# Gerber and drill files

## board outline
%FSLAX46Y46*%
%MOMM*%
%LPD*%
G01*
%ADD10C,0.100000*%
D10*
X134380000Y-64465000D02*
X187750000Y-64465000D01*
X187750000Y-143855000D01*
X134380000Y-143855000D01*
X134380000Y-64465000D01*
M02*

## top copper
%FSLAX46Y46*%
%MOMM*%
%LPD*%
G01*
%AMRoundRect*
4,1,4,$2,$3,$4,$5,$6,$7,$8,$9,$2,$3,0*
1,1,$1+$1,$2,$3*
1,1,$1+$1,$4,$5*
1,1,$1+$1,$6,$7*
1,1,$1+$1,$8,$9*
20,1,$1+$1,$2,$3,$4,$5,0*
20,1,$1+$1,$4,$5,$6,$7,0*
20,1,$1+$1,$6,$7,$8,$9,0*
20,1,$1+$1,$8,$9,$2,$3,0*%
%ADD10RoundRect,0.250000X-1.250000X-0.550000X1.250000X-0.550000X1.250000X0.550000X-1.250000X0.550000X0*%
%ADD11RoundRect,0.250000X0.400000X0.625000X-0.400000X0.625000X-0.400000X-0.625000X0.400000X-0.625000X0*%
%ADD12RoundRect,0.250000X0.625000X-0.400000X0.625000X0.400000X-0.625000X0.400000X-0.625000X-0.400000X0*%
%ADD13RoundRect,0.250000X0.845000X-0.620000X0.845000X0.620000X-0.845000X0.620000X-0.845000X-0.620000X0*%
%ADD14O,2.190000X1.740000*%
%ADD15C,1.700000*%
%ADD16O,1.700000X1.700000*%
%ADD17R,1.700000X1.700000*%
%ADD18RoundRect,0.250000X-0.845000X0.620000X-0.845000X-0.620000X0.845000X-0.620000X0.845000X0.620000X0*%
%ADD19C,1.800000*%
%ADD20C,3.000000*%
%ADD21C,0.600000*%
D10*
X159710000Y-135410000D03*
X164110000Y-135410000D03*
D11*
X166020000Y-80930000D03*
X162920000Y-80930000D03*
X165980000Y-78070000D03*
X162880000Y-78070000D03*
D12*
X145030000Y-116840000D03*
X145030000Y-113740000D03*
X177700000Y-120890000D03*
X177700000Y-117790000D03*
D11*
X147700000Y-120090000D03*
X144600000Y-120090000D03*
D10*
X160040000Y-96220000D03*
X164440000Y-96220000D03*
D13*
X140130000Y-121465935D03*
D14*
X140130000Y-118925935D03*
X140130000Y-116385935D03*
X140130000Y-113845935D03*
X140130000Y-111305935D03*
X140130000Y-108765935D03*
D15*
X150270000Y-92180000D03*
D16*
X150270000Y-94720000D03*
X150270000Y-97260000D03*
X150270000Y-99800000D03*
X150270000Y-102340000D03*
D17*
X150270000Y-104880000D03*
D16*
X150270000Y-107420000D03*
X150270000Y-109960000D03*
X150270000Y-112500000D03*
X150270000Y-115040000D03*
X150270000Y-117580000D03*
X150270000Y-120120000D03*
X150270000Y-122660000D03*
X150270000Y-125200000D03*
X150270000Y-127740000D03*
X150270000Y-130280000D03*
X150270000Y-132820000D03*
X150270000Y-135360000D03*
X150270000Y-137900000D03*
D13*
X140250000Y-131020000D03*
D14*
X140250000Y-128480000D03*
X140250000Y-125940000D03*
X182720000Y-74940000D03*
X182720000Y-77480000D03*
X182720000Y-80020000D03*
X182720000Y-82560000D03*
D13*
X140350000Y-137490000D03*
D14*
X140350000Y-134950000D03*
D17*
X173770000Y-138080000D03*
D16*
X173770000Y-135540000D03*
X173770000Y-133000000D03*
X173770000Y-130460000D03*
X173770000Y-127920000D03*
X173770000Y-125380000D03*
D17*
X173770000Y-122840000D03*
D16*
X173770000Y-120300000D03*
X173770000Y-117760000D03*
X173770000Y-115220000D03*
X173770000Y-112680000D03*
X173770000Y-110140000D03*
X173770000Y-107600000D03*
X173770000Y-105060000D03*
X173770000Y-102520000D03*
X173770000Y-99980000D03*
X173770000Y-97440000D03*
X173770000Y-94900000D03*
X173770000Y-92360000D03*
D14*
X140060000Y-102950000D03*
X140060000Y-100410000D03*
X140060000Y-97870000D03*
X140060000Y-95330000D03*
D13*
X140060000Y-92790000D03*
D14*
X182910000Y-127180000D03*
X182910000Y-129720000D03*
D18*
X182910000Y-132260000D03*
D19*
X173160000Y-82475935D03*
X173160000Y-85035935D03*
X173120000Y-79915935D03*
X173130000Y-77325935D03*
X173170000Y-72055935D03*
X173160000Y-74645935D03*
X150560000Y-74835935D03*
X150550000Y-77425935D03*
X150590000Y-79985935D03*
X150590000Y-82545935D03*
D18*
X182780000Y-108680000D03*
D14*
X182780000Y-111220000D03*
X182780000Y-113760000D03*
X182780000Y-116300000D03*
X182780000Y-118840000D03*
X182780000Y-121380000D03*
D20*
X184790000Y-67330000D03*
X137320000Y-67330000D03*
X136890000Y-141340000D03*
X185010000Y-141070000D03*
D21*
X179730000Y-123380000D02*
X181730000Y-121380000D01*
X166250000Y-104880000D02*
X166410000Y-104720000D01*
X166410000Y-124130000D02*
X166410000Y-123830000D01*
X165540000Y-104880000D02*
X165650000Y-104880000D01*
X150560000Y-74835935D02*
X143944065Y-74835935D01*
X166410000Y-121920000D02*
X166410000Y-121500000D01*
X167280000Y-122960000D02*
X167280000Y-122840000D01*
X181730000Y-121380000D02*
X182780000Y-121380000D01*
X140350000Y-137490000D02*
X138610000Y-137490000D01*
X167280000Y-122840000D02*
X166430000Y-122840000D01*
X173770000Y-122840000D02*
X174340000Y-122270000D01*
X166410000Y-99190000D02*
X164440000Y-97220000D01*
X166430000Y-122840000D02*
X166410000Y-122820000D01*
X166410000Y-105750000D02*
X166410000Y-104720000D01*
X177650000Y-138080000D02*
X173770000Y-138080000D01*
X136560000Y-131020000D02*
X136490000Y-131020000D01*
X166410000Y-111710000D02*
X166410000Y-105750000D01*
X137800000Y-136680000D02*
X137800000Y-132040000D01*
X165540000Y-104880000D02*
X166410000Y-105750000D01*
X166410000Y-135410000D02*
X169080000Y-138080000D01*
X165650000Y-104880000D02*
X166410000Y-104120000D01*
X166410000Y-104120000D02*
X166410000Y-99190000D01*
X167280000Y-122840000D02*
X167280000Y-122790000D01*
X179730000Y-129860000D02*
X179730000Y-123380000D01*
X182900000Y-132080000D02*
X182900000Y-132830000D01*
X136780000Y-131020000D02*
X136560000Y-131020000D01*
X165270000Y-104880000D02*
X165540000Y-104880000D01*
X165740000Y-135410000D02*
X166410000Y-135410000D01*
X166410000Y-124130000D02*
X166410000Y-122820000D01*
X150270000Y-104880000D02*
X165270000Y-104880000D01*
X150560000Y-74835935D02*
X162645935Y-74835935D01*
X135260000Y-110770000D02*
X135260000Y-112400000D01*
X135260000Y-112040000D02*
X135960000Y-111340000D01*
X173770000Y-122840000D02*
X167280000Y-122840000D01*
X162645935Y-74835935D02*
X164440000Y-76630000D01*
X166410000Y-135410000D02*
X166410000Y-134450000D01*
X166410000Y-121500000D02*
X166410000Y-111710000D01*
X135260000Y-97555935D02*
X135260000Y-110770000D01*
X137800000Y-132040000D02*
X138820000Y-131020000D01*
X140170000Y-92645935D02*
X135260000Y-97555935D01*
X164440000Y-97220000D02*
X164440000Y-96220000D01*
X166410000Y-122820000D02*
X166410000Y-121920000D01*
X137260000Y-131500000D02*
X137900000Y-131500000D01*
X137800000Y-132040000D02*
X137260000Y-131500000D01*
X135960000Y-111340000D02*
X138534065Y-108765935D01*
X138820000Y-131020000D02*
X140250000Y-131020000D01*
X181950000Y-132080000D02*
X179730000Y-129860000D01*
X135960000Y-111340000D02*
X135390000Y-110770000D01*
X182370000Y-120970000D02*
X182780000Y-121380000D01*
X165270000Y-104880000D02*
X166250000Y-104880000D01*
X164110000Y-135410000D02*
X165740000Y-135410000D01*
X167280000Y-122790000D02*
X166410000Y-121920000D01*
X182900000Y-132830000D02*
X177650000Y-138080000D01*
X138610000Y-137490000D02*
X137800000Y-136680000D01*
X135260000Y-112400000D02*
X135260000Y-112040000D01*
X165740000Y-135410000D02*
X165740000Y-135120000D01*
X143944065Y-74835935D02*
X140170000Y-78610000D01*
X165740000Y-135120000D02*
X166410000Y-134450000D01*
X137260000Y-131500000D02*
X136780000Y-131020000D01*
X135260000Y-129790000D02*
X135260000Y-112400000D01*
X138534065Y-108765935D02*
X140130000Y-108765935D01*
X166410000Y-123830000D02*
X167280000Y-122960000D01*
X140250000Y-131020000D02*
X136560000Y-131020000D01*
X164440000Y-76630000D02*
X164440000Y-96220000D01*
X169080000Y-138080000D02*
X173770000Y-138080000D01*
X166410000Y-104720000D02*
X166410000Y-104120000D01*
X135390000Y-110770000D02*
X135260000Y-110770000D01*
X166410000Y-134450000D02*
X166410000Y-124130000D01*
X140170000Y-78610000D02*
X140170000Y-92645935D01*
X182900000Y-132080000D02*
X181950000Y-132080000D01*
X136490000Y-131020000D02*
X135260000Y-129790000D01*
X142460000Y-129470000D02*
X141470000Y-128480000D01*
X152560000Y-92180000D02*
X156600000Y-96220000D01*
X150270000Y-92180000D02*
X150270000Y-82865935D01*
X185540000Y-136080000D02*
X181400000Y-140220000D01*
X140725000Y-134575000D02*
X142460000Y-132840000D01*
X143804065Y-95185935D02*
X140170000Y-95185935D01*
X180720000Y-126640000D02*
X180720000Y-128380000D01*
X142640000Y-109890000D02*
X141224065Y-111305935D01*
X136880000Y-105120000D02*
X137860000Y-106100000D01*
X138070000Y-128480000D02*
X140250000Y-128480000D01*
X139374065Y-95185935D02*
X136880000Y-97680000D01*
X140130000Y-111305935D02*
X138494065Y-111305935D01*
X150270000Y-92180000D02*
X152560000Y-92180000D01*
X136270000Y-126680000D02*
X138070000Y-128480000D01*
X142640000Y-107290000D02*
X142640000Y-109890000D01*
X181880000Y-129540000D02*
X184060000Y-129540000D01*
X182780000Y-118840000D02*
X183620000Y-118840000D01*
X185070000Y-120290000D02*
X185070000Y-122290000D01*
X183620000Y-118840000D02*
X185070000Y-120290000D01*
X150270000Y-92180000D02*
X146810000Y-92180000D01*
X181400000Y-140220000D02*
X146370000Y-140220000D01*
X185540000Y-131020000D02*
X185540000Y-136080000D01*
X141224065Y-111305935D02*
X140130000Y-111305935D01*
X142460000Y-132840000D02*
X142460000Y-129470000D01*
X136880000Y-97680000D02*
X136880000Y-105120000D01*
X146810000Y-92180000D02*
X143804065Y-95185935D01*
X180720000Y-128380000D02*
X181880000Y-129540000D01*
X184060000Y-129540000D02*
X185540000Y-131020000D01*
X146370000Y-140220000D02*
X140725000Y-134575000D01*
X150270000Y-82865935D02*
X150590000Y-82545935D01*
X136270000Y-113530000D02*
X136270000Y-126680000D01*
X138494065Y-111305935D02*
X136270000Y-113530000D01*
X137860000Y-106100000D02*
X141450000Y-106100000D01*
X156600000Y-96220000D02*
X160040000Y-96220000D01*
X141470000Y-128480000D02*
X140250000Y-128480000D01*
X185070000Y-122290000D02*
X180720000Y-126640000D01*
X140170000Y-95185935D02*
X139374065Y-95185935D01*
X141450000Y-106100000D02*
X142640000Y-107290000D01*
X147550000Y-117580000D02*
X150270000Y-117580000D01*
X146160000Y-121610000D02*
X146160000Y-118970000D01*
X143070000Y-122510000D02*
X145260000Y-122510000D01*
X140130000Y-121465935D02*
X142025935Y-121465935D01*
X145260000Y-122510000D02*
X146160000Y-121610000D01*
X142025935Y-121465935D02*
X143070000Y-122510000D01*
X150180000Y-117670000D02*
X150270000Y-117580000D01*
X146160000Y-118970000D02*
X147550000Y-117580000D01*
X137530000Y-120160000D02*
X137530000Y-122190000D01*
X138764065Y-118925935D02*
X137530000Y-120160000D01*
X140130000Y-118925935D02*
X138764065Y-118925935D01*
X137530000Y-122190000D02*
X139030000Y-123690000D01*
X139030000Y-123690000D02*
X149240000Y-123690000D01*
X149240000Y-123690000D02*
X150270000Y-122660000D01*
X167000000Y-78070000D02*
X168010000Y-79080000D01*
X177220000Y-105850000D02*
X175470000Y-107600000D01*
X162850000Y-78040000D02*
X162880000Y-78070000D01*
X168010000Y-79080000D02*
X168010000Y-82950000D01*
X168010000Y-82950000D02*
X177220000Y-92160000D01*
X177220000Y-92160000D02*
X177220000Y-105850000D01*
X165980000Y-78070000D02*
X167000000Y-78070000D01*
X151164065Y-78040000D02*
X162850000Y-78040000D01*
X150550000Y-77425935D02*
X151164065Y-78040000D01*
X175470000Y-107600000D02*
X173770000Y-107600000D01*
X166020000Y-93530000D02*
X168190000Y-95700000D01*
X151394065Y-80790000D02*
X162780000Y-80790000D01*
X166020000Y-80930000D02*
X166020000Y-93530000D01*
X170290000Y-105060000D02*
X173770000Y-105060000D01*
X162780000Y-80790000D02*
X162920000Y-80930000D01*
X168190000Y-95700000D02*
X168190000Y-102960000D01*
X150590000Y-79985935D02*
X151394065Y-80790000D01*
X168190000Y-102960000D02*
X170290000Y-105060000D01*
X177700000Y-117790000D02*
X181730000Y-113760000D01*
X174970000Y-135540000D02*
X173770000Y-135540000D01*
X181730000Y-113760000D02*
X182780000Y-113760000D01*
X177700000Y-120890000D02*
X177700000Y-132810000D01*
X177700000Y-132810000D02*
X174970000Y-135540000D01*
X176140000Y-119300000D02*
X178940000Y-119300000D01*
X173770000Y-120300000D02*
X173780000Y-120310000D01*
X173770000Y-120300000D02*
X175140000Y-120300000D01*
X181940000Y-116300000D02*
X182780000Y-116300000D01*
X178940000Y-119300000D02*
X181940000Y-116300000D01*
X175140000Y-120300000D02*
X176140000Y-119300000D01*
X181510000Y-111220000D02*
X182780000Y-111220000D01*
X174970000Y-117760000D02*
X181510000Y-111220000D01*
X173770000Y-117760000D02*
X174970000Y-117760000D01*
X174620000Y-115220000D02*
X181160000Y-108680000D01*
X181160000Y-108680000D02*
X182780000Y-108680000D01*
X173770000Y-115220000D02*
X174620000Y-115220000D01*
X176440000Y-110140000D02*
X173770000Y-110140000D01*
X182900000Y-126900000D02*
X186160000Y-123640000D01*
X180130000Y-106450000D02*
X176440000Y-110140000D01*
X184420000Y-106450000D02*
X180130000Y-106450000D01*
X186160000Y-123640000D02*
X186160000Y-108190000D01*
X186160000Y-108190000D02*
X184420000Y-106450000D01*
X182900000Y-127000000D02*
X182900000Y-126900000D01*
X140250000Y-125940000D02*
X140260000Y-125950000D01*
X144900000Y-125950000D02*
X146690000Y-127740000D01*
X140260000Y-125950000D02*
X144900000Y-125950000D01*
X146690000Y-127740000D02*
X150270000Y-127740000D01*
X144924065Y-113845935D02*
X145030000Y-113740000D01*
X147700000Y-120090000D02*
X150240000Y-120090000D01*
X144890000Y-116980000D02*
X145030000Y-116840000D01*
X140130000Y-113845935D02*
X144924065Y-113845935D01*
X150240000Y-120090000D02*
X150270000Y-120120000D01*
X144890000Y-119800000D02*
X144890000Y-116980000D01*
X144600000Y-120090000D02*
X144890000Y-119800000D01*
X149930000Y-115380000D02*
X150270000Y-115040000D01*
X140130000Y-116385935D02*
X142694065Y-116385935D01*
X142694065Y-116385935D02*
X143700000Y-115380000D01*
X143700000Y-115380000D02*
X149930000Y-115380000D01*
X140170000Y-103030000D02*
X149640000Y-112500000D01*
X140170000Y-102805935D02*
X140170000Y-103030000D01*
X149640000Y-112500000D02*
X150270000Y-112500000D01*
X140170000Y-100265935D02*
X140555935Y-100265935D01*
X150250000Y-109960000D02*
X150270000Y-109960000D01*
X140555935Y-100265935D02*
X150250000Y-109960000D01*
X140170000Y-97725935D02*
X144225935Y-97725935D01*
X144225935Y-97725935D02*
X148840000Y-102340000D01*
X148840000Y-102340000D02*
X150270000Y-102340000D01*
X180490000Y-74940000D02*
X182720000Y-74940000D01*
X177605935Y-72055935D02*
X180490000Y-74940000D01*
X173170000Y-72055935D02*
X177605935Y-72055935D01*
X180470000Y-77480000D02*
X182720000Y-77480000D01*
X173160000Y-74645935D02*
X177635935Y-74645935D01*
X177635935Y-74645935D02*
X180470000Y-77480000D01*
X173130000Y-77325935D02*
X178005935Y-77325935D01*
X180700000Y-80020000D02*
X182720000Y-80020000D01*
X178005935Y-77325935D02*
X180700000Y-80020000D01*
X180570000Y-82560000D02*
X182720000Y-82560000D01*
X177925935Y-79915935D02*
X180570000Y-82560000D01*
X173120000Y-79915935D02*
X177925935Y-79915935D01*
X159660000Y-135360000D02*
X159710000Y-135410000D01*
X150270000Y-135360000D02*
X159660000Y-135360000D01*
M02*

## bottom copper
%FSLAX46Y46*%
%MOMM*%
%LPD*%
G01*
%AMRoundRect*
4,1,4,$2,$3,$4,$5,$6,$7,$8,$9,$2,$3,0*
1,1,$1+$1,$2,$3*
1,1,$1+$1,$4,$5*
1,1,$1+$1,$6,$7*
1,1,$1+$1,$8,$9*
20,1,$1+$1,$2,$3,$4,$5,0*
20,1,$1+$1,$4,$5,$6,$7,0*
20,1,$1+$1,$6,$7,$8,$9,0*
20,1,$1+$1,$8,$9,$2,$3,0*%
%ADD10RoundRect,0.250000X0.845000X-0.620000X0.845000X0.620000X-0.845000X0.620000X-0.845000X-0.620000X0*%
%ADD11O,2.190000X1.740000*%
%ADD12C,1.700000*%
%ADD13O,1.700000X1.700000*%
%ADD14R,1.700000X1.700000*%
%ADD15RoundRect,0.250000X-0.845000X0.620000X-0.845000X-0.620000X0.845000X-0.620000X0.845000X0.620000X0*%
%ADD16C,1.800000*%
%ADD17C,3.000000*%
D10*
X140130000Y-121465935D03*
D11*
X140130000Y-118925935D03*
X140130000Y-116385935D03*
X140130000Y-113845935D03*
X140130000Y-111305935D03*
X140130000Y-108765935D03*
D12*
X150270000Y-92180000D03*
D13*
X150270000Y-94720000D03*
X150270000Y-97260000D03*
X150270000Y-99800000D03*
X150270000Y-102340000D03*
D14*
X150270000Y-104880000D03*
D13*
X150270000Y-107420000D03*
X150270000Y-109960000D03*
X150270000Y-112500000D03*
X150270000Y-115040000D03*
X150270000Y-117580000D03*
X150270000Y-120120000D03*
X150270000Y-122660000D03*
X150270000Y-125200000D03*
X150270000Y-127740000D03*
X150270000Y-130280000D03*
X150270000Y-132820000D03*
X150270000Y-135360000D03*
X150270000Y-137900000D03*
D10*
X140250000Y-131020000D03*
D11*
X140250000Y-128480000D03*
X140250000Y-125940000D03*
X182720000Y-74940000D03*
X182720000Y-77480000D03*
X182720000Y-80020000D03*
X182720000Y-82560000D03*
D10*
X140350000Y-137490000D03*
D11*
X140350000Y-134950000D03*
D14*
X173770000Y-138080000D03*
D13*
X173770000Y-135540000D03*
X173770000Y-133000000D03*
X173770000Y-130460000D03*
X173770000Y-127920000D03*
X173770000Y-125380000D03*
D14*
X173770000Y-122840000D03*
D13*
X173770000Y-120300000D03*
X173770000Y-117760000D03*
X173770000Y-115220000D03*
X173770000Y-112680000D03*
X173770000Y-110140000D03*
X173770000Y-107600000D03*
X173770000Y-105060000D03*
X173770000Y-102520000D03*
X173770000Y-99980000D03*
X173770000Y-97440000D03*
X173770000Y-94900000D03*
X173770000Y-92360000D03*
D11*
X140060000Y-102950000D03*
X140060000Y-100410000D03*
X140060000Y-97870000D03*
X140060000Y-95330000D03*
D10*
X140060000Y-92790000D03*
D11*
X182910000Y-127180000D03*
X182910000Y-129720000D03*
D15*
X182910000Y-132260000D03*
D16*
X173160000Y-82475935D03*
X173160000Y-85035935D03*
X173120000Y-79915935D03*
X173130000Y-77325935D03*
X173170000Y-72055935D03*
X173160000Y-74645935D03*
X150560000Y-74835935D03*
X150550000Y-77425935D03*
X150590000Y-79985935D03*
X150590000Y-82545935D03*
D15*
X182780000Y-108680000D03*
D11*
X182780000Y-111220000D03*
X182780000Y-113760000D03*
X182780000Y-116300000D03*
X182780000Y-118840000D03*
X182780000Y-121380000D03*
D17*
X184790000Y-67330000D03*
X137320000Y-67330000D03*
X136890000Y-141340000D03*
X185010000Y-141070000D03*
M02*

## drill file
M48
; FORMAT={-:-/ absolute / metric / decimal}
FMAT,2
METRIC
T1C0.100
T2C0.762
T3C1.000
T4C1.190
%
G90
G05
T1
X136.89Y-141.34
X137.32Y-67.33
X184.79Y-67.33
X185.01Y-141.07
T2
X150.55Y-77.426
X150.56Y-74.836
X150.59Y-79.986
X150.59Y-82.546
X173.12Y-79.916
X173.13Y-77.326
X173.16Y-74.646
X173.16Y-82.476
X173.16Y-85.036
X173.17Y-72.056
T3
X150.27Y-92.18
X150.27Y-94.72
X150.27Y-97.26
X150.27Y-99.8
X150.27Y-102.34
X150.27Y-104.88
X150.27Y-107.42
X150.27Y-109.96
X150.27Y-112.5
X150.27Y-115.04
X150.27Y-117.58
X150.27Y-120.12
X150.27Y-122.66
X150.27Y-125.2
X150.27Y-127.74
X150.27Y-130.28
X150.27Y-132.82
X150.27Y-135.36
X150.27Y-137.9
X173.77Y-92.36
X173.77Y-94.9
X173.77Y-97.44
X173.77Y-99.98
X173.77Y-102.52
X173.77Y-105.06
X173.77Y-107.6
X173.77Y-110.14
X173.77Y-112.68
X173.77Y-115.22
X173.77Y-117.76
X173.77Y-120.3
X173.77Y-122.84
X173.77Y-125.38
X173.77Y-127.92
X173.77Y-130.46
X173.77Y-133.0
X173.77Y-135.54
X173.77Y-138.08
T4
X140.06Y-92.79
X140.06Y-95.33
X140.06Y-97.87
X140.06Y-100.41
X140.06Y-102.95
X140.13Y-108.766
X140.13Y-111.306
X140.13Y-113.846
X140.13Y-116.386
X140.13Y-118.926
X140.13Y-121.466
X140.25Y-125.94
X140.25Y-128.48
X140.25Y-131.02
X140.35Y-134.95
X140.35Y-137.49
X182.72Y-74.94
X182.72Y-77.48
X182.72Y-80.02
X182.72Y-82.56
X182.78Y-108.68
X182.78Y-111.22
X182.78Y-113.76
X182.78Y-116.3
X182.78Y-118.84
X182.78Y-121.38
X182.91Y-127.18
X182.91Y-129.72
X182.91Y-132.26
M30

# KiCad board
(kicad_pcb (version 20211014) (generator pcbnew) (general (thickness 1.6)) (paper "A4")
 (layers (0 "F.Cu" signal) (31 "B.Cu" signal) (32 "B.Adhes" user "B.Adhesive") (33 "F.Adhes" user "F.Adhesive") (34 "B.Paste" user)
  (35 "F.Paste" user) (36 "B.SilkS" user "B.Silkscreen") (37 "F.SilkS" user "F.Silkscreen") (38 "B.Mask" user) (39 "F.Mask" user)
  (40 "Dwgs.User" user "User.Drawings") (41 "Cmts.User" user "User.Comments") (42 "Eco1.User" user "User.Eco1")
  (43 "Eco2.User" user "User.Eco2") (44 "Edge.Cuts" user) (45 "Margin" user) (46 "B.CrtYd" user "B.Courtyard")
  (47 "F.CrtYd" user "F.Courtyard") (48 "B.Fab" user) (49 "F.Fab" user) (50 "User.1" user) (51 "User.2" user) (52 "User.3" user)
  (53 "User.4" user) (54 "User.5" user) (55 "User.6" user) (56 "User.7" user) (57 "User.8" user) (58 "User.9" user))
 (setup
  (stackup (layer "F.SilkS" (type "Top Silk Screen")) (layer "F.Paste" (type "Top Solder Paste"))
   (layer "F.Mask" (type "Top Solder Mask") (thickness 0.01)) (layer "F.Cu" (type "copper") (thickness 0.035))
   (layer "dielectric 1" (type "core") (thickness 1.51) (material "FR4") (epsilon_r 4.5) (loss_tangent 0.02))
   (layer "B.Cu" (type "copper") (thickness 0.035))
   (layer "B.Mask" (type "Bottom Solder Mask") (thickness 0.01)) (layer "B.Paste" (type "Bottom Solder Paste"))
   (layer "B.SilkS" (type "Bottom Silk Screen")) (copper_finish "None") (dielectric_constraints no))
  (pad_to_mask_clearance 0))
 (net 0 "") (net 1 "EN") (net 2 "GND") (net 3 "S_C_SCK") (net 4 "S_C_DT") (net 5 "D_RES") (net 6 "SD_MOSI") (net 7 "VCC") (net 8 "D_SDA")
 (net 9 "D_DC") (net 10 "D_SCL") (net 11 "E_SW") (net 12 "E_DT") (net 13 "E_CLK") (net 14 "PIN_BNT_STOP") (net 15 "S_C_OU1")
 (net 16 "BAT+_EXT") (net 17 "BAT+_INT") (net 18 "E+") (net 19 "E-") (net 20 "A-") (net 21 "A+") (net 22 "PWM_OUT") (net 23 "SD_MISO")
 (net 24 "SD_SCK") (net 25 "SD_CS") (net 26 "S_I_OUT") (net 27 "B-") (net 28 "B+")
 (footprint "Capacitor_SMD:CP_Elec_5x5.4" (layer "F.Cu") (at 161.91 135.41)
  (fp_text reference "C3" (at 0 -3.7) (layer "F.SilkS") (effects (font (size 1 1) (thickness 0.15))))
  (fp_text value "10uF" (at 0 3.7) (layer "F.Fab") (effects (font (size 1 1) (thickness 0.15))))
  (pad "1" smd roundrect (at -2.2 0) (size 3 1.6) (layers "F.Cu" "F.Paste" "F.Mask") (roundrect_rratio 0.15625) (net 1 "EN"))
  (pad "2" smd roundrect (at 2.2 0) (size 3 1.6) (layers "F.Cu" "F.Paste" "F.Mask") (roundrect_rratio 0.15625) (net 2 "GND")))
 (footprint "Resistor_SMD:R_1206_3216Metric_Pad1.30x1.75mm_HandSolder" (layer "F.Cu") (at 164.47 80.93 180)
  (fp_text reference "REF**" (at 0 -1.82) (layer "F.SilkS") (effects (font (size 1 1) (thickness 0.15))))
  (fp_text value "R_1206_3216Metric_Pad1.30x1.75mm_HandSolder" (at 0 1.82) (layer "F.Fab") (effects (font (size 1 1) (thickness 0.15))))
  (pad "1" smd roundrect (at -1.55 0 180) (size 1.3 1.75) (layers "F.Cu" "F.Paste" "F.Mask") (roundrect_rratio 0.192308) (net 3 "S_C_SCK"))
  (pad "2" smd roundrect (at 1.55 0 180) (size 1.3 1.75) (layers "F.Cu" "F.Paste" "F.Mask") (roundrect_rratio 0.192308) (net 3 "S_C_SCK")))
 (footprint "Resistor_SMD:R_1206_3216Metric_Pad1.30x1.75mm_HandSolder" (layer "F.Cu") (at 164.43 78.07 180)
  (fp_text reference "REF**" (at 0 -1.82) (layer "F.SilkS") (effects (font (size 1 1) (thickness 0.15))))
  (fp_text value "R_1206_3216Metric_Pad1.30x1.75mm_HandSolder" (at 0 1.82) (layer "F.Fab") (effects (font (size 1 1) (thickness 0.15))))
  (pad "1" smd roundrect (at -1.55 0 180) (size 1.3 1.75) (layers "F.Cu" "F.Paste" "F.Mask") (roundrect_rratio 0.192308) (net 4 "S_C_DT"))
  (pad "2" smd roundrect (at 1.55 0 180) (size 1.3 1.75) (layers "F.Cu" "F.Paste" "F.Mask") (roundrect_rratio 0.192308) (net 4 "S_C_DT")))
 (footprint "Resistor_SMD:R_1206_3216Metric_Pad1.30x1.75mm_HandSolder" (layer "F.Cu") (at 145.03 115.29 90)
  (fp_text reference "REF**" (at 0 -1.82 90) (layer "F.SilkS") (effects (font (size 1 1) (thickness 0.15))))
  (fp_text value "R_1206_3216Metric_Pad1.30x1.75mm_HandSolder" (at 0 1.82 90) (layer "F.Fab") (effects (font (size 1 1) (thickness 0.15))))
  (pad "1" smd roundrect (at -1.55 0 90) (size 1.3 1.75) (layers "F.Cu" "F.Paste" "F.Mask") (roundrect_rratio 0.192308) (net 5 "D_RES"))
  (pad "2" smd roundrect (at 1.55 0 90) (size 1.3 1.75) (layers "F.Cu" "F.Paste" "F.Mask") (roundrect_rratio 0.192308) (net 5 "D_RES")))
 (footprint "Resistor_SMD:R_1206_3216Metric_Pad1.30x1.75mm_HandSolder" (layer "F.Cu") (at 177.7 119.34 90)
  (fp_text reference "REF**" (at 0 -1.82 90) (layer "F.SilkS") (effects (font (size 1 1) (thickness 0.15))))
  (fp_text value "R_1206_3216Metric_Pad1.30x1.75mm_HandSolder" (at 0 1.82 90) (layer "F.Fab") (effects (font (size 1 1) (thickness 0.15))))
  (pad "1" smd roundrect (at -1.55 0 90) (size 1.3 1.75) (layers "F.Cu" "F.Paste" "F.Mask") (roundrect_rratio 0.192308) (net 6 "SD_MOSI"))
  (pad "2" smd roundrect (at 1.55 0 90) (size 1.3 1.75) (layers "F.Cu" "F.Paste" "F.Mask") (roundrect_rratio 0.192308) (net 6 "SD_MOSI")))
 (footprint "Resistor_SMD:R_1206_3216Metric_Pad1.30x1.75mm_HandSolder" (layer "F.Cu") (at 146.15 120.09 180)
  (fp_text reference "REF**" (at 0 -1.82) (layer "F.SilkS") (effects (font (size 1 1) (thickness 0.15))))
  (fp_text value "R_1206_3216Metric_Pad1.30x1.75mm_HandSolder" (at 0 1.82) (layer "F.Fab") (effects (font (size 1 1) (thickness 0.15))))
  (pad "1" smd roundrect (at -1.55 0 180) (size 1.3 1.75) (layers "F.Cu" "F.Paste" "F.Mask") (roundrect_rratio 0.192308) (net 5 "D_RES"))
  (pad "2" smd roundrect (at 1.55 0 180) (size 1.3 1.75) (layers "F.Cu" "F.Paste" "F.Mask") (roundrect_rratio 0.192308) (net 5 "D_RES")))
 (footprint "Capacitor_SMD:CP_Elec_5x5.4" (layer "F.Cu") (at 162.24 96.22)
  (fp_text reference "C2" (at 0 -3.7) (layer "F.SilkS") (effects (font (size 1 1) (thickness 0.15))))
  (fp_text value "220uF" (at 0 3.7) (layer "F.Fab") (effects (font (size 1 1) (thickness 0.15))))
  (pad "1" smd roundrect (at -2.2 0) (size 3 1.6) (layers "F.Cu" "F.Paste" "F.Mask") (roundrect_rratio 0.15625) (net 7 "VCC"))
  (pad "2" smd roundrect (at 2.2 0) (size 3 1.6) (layers "F.Cu" "F.Paste" "F.Mask") (roundrect_rratio 0.15625) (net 2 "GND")))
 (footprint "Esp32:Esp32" (layer "F.Cu") (at 162.18 114.97)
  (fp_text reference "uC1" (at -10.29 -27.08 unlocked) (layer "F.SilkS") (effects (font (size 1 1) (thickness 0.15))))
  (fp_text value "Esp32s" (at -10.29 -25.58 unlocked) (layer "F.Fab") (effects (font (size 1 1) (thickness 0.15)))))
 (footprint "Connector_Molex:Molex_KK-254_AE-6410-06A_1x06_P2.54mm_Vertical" (layer "B.Cu") (at 140.13 121.465935 90)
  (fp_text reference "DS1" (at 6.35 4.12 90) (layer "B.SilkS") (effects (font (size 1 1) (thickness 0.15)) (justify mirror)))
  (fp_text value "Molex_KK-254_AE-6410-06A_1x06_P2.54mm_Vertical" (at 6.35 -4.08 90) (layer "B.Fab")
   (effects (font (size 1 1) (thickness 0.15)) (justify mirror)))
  (pad "1" thru_hole roundrect (at 0 0 90) (size 1.74 2.19) (drill 1.19) (layers *.Cu *.Mask) (roundrect_rratio 0.143678) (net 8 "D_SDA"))
  (pad "2" thru_hole oval (at 2.54 0 90) (size 1.74 2.19) (drill 1.19) (layers *.Cu *.Mask) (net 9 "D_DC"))
  (pad "3" thru_hole oval (at 5.08 0 90) (size 1.74 2.19) (drill 1.19) (layers *.Cu *.Mask) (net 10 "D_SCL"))
  (pad "4" thru_hole oval (at 7.62 0 90) (size 1.74 2.19) (drill 1.19) (layers *.Cu *.Mask) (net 5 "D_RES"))
  (pad "5" thru_hole oval (at 10.16 0 90) (size 1.74 2.19) (drill 1.19) (layers *.Cu *.Mask) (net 7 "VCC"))
  (pad "6" thru_hole oval (at 12.7 0 90) (size 1.74 2.19) (drill 1.19) (layers *.Cu *.Mask) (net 2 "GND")))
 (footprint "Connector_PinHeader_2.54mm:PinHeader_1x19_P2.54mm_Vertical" (layer "B.Cu") (at 150.27 92.18 180)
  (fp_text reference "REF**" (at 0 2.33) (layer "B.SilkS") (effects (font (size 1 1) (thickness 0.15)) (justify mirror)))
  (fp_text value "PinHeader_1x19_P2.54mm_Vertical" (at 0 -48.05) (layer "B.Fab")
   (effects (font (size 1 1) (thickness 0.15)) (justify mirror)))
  (pad "1" thru_hole circle (at 0 0 180) (size 1.7 1.7) (drill 1) (layers *.Cu *.Mask) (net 7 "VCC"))
  (pad "2" thru_hole oval (at 0 -2.54 180) (size 1.7 1.7) (drill 1) (layers *.Cu *.Mask))
  (pad "3" thru_hole oval (at 0 -5.08 180) (size 1.7 1.7) (drill 1) (layers *.Cu *.Mask))
  (pad "4" thru_hole oval (at 0 -7.62 180) (size 1.7 1.7) (drill 1) (layers *.Cu *.Mask))
  (pad "5" thru_hole oval (at 0 -10.16 180) (size 1.7 1.7) (drill 1) (layers *.Cu *.Mask) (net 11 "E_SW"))
  (pad "6" thru_hole rect (at 0 -12.7 180) (size 1.7 1.7) (drill 1) (layers *.Cu *.Mask) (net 2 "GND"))
  (pad "7" thru_hole oval (at 0 -15.24 180) (size 1.7 1.7) (drill 1) (layers *.Cu *.Mask))
  (pad "8" thru_hole oval (at 0 -17.78 180) (size 1.7 1.7) (drill 1) (layers *.Cu *.Mask) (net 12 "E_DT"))
  (pad "9" thru_hole oval (at 0 -20.32 180) (size 1.7 1.7) (drill 1) (layers *.Cu *.Mask) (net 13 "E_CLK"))
  (pad "10" thru_hole oval (at 0 -22.86 180) (size 1.7 1.7) (drill 1) (layers *.Cu *.Mask) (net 10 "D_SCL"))
  (pad "11" thru_hole oval (at 0 -25.4 180) (size 1.7 1.7) (drill 1) (layers *.Cu *.Mask) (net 8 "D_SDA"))
  (pad "12" thru_hole oval (at 0 -27.94 180) (size 1.7 1.7) (drill 1) (layers *.Cu *.Mask) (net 5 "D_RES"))
  (pad "13" thru_hole oval (at 0 -30.48 180) (size 1.7 1.7) (drill 1) (layers *.Cu *.Mask) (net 9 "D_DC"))
  (pad "14" thru_hole oval (at 0 -33.02 180) (size 1.7 1.7) (drill 1) (layers *.Cu *.Mask) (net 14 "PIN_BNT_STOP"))
  (pad "15" thru_hole oval (at 0 -35.56 180) (size 1.7 1.7) (drill 1) (layers *.Cu *.Mask) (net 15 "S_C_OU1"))
  (pad "16" thru_hole oval (at 0 -38.1 180) (size 1.7 1.7) (drill 1) (layers *.Cu *.Mask) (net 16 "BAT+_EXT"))
  (pad "17" thru_hole oval (at 0 -40.64 180) (size 1.7 1.7) (drill 1) (layers *.Cu *.Mask) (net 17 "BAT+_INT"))
  (pad "18" thru_hole oval (at 0 -43.18 180) (size 1.7 1.7) (drill 1) (layers *.Cu *.Mask) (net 1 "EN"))
  (pad "19" thru_hole oval (at 0 -45.72 180) (size 1.7 1.7) (drill 1) (layers *.Cu *.Mask)))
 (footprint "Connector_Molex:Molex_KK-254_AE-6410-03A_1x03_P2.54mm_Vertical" (layer "B.Cu") (at 140.25 131.02 90)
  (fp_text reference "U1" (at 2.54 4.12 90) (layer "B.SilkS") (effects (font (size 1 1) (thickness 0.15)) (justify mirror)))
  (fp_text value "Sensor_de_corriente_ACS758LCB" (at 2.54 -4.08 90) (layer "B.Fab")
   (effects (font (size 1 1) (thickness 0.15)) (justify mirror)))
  (pad "1" thru_hole roundrect (at 0 0 90) (size 1.74 2.19) (drill 1.19) (layers *.Cu *.Mask) (roundrect_rratio 0.143678) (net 2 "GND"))
  (pad "2" thru_hole oval (at 2.54 0 90) (size 1.74 2.19) (drill 1.19) (layers *.Cu *.Mask) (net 7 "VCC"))
  (pad "3" thru_hole oval (at 5.08 0 90) (size 1.74 2.19) (drill 1.19) (layers *.Cu *.Mask) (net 15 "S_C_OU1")))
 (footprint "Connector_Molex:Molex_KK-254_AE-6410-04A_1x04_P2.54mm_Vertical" (layer "B.Cu") (at 182.72 74.94 -90)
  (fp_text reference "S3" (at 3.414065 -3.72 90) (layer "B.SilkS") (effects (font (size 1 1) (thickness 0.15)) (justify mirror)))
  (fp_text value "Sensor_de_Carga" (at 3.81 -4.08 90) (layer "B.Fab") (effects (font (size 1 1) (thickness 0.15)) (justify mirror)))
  (pad "1" thru_hole oval (at 0 0 270) (size 1.74 2.19) (drill 1.19) (layers *.Cu *.Mask) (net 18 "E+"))
  (pad "2" thru_hole oval (at 2.54 0 270) (size 1.74 2.19) (drill 1.19) (layers *.Cu *.Mask) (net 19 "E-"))
  (pad "3" thru_hole oval (at 5.08 0 270) (size 1.74 2.19) (drill 1.19) (layers *.Cu *.Mask) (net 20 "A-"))
  (pad "4" thru_hole oval (at 7.62 0 270) (size 1.74 2.19) (drill 1.19) (layers *.Cu *.Mask) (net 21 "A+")))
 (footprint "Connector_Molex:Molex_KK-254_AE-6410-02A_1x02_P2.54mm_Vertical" (layer "B.Cu") (at 140.35 137.49 90)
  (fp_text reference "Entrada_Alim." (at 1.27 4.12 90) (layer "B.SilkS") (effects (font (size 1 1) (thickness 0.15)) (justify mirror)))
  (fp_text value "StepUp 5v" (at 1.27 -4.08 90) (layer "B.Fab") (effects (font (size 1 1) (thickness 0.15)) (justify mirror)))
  (pad "1" thru_hole roundrect (at 0 0 90) (size 1.74 2.19) (drill 1.19) (layers *.Cu *.Mask) (roundrect_rratio 0.143678) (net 2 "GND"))
  (pad "2" thru_hole oval (at 2.54 0 90) (size 1.74 2.19) (drill 1.19) (layers *.Cu *.Mask) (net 7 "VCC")))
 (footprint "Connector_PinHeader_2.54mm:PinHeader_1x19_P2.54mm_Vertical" (layer "B.Cu") (at 173.77 138.08)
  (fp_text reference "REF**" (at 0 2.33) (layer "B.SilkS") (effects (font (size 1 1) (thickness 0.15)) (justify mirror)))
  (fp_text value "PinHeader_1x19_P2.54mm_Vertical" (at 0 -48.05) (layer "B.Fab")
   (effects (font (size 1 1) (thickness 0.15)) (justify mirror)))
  (pad "1" thru_hole rect (at 0 0) (size 1.7 1.7) (drill 1) (layers *.Cu *.Mask) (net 2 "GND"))
  (pad "2" thru_hole oval (at 0 -2.54) (size 1.7 1.7) (drill 1) (layers *.Cu *.Mask) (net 6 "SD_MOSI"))
  (pad "3" thru_hole oval (at 0 -5.08) (size 1.7 1.7) (drill 1) (layers *.Cu *.Mask) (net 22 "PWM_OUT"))
  (pad "4" thru_hole oval (at 0 -7.62) (size 1.7 1.7) (drill 1) (layers *.Cu *.Mask))
  (pad "5" thru_hole oval (at 0 -10.16) (size 1.7 1.7) (drill 1) (layers *.Cu *.Mask))
  (pad "6" thru_hole oval (at 0 -12.7) (size 1.7 1.7) (drill 1) (layers *.Cu *.Mask))
  (pad "7" thru_hole rect (at 0 -15.24) (size 1.7 1.7) (drill 1) (layers *.Cu *.Mask) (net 2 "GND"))
  (pad "8" thru_hole oval (at 0 -17.78) (size 1.7 1.7) (drill 1) (layers *.Cu *.Mask) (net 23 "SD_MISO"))
  (pad "9" thru_hole oval (at 0 -20.32) (size 1.7 1.7) (drill 1) (layers *.Cu *.Mask) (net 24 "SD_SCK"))
  (pad "10" thru_hole oval (at 0 -22.86) (size 1.7 1.7) (drill 1) (layers *.Cu *.Mask) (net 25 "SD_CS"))
  (pad "11" thru_hole oval (at 0 -25.4) (size 1.7 1.7) (drill 1) (layers *.Cu *.Mask))
  (pad "12" thru_hole oval (at 0 -27.94) (size 1.7 1.7) (drill 1) (layers *.Cu *.Mask) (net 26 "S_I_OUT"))
  (pad "13" thru_hole oval (at 0 -30.48) (size 1.7 1.7) (drill 1) (layers *.Cu *.Mask) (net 4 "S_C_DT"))
  (pad "14" thru_hole oval (at 0 -33.02) (size 1.7 1.7) (drill 1) (layers *.Cu *.Mask) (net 3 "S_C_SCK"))
  (pad "15" thru_hole oval (at 0 -35.56) (size 1.7 1.7) (drill 1) (layers *.Cu *.Mask))
  (pad "16" thru_hole oval (at 0 -38.1) (size 1.7 1.7) (drill 1) (layers *.Cu *.Mask))
  (pad "17" thru_hole oval (at 0 -40.64) (size 1.7 1.7) (drill 1) (layers *.Cu *.Mask))
  (pad "18" thru_hole oval (at 0 -43.18) (size 1.7 1.7) (drill 1) (layers *.Cu *.Mask))
  (pad "19" thru_hole oval (at 0 -45.72) (size 1.7 1.7) (drill 1) (layers *.Cu *.Mask)))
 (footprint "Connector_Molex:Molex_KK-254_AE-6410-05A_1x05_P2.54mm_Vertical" (layer "B.Cu") (at 140.06 102.95 90)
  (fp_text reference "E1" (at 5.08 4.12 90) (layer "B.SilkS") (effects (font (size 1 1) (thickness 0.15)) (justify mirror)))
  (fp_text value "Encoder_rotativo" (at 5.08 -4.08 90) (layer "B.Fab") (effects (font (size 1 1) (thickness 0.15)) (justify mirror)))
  (pad "1" thru_hole oval (at 0 0 90) (size 1.74 2.19) (drill 1.19) (layers *.Cu *.Mask) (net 13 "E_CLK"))
  (pad "2" thru_hole oval (at 2.54 0 90) (size 1.74 2.19) (drill 1.19) (layers *.Cu *.Mask) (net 12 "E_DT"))
  (pad "3" thru_hole oval (at 5.08 0 90) (size 1.74 2.19) (drill 1.19) (layers *.Cu *.Mask) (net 11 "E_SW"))
  (pad "4" thru_hole oval (at 7.62 0 90) (size 1.74 2.19) (drill 1.19) (layers *.Cu *.Mask) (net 7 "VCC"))
  (pad "5" thru_hole roundrect (at 10.16 0 90) (size 1.74 2.19) (drill 1.19) (layers *.Cu *.Mask) (roundrect_rratio 0.143678) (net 2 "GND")))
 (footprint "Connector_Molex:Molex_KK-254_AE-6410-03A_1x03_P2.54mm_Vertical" (layer "B.Cu") (at 182.91 127.18 -90)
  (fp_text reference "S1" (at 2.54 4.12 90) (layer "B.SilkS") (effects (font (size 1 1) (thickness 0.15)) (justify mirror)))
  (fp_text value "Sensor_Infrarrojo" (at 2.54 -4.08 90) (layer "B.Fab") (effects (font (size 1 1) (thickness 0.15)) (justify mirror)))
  (pad "1" thru_hole oval (at 0 0 270) (size 1.74 2.19) (drill 1.19) (layers *.Cu *.Mask) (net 26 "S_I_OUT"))
  (pad "2" thru_hole oval (at 2.54 0 270) (size 1.74 2.19) (drill 1.19) (layers *.Cu *.Mask) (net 7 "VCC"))
  (pad "3" thru_hole roundrect (at 5.08 0 270) (size 1.74 2.19) (drill 1.19) (layers *.Cu *.Mask) (roundrect_rratio 0.143678) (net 2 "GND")))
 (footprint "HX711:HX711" (layer "B.Cu") (at 161.38 78.605935 180)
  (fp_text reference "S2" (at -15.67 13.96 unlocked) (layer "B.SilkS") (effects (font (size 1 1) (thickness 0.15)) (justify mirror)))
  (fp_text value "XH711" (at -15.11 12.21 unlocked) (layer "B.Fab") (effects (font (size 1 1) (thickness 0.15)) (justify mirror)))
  (pad "" thru_hole circle (at -11.78 -3.87 90) (size 1.8 1.8) (drill 0.762) (layers *.Cu *.Mask) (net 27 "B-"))
  (pad "" thru_hole circle (at -11.78 -6.43 90) (size 1.8 1.8) (drill 0.762) (layers *.Cu *.Mask) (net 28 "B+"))
  (pad "1" thru_hole circle (at -11.74 -1.31 90) (size 1.8 1.8) (drill 0.762) (layers *.Cu *.Mask) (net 21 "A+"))
  (pad "2" thru_hole circle (at -11.75 1.28 90) (size 1.8 1.8) (drill 0.762) (layers *.Cu *.Mask) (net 20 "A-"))
  (pad "3" thru_hole circle (at -11.79 6.55 90) (size 1.8 1.8) (drill 0.762) (layers *.Cu *.Mask) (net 18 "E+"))
  (pad "4" thru_hole circle (at -11.78 3.96 90) (size 1.8 1.8) (drill 0.762) (layers *.Cu *.Mask) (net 19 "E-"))
  (pad "5" thru_hole circle (at 10.82 3.77 90) (size 1.8 1.8) (drill 0.762) (layers *.Cu *.Mask) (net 2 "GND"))
  (pad "6" thru_hole circle (at 10.83 1.18 90) (size 1.8 1.8) (drill 0.762) (layers *.Cu *.Mask) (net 4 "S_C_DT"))
  (pad "7" thru_hole circle (at 10.79 -1.38 90) (size 1.8 1.8) (drill 0.762) (layers *.Cu *.Mask) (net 3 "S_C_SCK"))
  (pad "8" thru_hole circle (at 10.79 -3.94 90) (size 1.8 1.8) (drill 0.762) (layers *.Cu *.Mask) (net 7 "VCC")))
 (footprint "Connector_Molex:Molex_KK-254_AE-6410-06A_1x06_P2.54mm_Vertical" (layer "B.Cu") (at 182.78 108.68 -90)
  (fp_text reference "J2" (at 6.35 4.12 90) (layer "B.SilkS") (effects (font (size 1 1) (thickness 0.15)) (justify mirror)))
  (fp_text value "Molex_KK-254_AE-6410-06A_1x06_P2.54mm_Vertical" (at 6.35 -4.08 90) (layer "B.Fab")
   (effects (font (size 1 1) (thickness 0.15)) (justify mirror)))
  (pad "1" thru_hole roundrect (at 0 0 270) (size 1.74 2.19) (drill 1.19) (layers *.Cu *.Mask) (roundrect_rratio 0.143678) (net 25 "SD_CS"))
  (pad "2" thru_hole oval (at 2.54 0 270) (size 1.74 2.19) (drill 1.19) (layers *.Cu *.Mask) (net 24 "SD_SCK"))
  (pad "3" thru_hole oval (at 5.08 0 270) (size 1.74 2.19) (drill 1.19) (layers *.Cu *.Mask) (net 6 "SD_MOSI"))
  (pad "4" thru_hole oval (at 7.62 0 270) (size 1.74 2.19) (drill 1.19) (layers *.Cu *.Mask) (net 23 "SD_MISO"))
  (pad "5" thru_hole oval (at 10.16 0 270) (size 1.74 2.19) (drill 1.19) (layers *.Cu *.Mask) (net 7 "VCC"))
  (pad "6" thru_hole oval (at 12.7 0 270) (size 1.74 2.19) (drill 1.19) (layers *.Cu *.Mask) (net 2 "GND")))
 (gr_rect (start 187.75 64.465) (end 134.38 143.855) (layer "Edge.Cuts") (width 0.1) (fill none))
 (via (at 184.79 67.33) (size 3) (drill 0.1) (layers "F.Cu" "B.Cu") (free) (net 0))
 (via (at 137.32 67.33) (size 3) (drill 0.1) (layers "F.Cu" "B.Cu") (free) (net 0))
 (via (at 136.89 141.34) (size 3) (drill 0.1) (layers "F.Cu" "B.Cu") (free) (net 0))
 (via (at 185.01 141.07) (size 3) (drill 0.1) (layers "F.Cu" "B.Cu") (free) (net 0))
 (segment (start 179.73 123.38) (end 181.73 121.38) (width 0.6) (layer "F.Cu") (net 2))
 (segment (start 166.25 104.88) (end 166.41 104.72) (width 0.6) (layer "F.Cu") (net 2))
 (segment (start 166.41 124.13) (end 166.41 123.83) (width 0.6) (layer "F.Cu") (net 2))
 (segment (start 165.54 104.88) (end 165.65 104.88) (width 0.6) (layer "F.Cu") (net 2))
 (segment (start 150.56 74.835935) (end 143.944065 74.835935) (width 0.6) (layer "F.Cu") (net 2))
 (segment (start 166.41 121.92) (end 166.41 121.5) (width 0.6) (layer "F.Cu") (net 2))
 (segment (start 167.28 122.96) (end 167.28 122.84) (width 0.6) (layer "F.Cu") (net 2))
 (segment (start 181.73 121.38) (end 182.78 121.38) (width 0.6) (layer "F.Cu") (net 2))
 (segment (start 140.35 137.49) (end 138.61 137.49) (width 0.6) (layer "F.Cu") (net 2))
 (segment (start 167.28 122.84) (end 166.43 122.84) (width 0.6) (layer "F.Cu") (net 2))
 (segment (start 173.77 122.84) (end 174.34 122.27) (width 0.6) (layer "F.Cu") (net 2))
 (segment (start 166.41 99.19) (end 164.44 97.22) (width 0.6) (layer "F.Cu") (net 2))
 (segment (start 166.43 122.84) (end 166.41 122.82) (width 0.6) (layer "F.Cu") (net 2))
 (segment (start 166.41 105.75) (end 166.41 104.72) (width 0.6) (layer "F.Cu") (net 2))
 (segment (start 177.65 138.08) (end 173.77 138.08) (width 0.6) (layer "F.Cu") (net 2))
 (segment (start 136.56 131.02) (end 136.49 131.02) (width 0.6) (layer "F.Cu") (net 2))
 (segment (start 166.41 111.71) (end 166.41 105.75) (width 0.6) (layer "F.Cu") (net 2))
 (segment (start 137.8 136.68) (end 137.8 132.04) (width 0.6) (layer "F.Cu") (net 2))
 (segment (start 165.54 104.88) (end 166.41 105.75) (width 0.6) (layer "F.Cu") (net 2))
 (segment (start 166.41 135.41) (end 169.08 138.08) (width 0.6) (layer "F.Cu") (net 2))
 (segment (start 165.65 104.88) (end 166.41 104.12) (width 0.6) (layer "F.Cu") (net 2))
 (segment (start 166.41 104.12) (end 166.41 99.19) (width 0.6) (layer "F.Cu") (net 2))
 (segment (start 167.28 122.84) (end 167.28 122.79) (width 0.6) (layer "F.Cu") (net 2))
 (segment (start 179.73 129.86) (end 179.73 123.38) (width 0.6) (layer "F.Cu") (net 2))
 (segment (start 182.9 132.08) (end 182.9 132.83) (width 0.6) (layer "F.Cu") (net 2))
 (segment (start 136.78 131.02) (end 136.56 131.02) (width 0.6) (layer "F.Cu") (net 2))
 (segment (start 165.27 104.88) (end 165.54 104.88) (width 0.6) (layer "F.Cu") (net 2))
 (segment (start 165.74 135.41) (end 166.41 135.41) (width 0.6) (layer "F.Cu") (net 2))
 (segment (start 166.41 124.13) (end 166.41 122.82) (width 0.6) (layer "F.Cu") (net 2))
 (segment (start 150.27 104.88) (end 165.27 104.88) (width 0.6) (layer "F.Cu") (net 2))
 (segment (start 150.56 74.835935) (end 162.645935 74.835935) (width 0.6) (layer "F.Cu") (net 2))
 (segment (start 135.26 110.77) (end 135.26 112.4) (width 0.6) (layer "F.Cu") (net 2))
 (segment (start 135.26 112.04) (end 135.96 111.34) (width 0.6) (layer "F.Cu") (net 2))
 (segment (start 173.77 122.84) (end 167.28 122.84) (width 0.6) (layer "F.Cu") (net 2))
 (segment (start 162.645935 74.835935) (end 164.44 76.63) (width 0.6) (layer "F.Cu") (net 2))
 (segment (start 166.41 135.41) (end 166.41 134.45) (width 0.6) (layer "F.Cu") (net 2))
 (segment (start 166.41 121.5) (end 166.41 111.71) (width 0.6) (layer "F.Cu") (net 2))
 (segment (start 135.26 97.555935) (end 135.26 110.77) (width 0.6) (layer "F.Cu") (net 2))
 (segment (start 137.8 132.04) (end 138.82 131.02) (width 0.6) (layer "F.Cu") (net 2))
 (segment (start 140.17 92.645935) (end 135.26 97.555935) (width 0.6) (layer "F.Cu") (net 2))
 (segment (start 164.44 97.22) (end 164.44 96.22) (width 0.6) (layer "F.Cu") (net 2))
 (segment (start 166.41 122.82) (end 166.41 121.92) (width 0.6) (layer "F.Cu") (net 2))
 (segment (start 137.26 131.5) (end 137.9 131.5) (width 0.6) (layer "F.Cu") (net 2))
 (segment (start 137.8 132.04) (end 137.26 131.5) (width 0.6) (layer "F.Cu") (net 2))
 (segment (start 135.96 111.34) (end 138.534065 108.765935) (width 0.6) (layer "F.Cu") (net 2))
 (segment (start 138.82 131.02) (end 140.25 131.02) (width 0.6) (layer "F.Cu") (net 2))
 (segment (start 181.95 132.08) (end 179.73 129.86) (width 0.6) (layer "F.Cu") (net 2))
 (segment (start 135.96 111.34) (end 135.39 110.77) (width 0.6) (layer "F.Cu") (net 2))
 (segment (start 182.37 120.97) (end 182.78 121.38) (width 0.6) (layer "F.Cu") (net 2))
 (segment (start 165.27 104.88) (end 166.25 104.88) (width 0.6) (layer "F.Cu") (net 2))
 (segment (start 164.11 135.41) (end 165.74 135.41) (width 0.6) (layer "F.Cu") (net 2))
 (segment (start 167.28 122.79) (end 166.41 121.92) (width 0.6) (layer "F.Cu") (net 2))
 (segment (start 182.9 132.83) (end 177.65 138.08) (width 0.6) (layer "F.Cu") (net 2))
 (segment (start 138.61 137.49) (end 137.8 136.68) (width 0.6) (layer "F.Cu") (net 2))
 (segment (start 135.26 112.4) (end 135.26 112.04) (width 0.6) (layer "F.Cu") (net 2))
 (segment (start 165.74 135.41) (end 165.74 135.12) (width 0.6) (layer "F.Cu") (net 2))
 (segment (start 143.944065 74.835935) (end 140.17 78.61) (width 0.6) (layer "F.Cu") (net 2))
 (segment (start 165.74 135.12) (end 166.41 134.45) (width 0.6) (layer "F.Cu") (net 2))
 (segment (start 137.26 131.5) (end 136.78 131.02) (width 0.6) (layer "F.Cu") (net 2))
 (segment (start 135.26 129.79) (end 135.26 112.4) (width 0.6) (layer "F.Cu") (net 2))
 (segment (start 138.534065 108.765935) (end 140.13 108.765935) (width 0.6) (layer "F.Cu") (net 2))
 (segment (start 166.41 123.83) (end 167.28 122.96) (width 0.6) (layer "F.Cu") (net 2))
 (segment (start 140.25 131.02) (end 136.56 131.02) (width 0.6) (layer "F.Cu") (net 2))
 (segment (start 164.44 76.63) (end 164.44 96.22) (width 0.6) (layer "F.Cu") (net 2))
 (segment (start 169.08 138.08) (end 173.77 138.08) (width 0.6) (layer "F.Cu") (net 2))
 (segment (start 166.41 104.72) (end 166.41 104.12) (width 0.6) (layer "F.Cu") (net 2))
 (segment (start 135.39 110.77) (end 135.26 110.77) (width 0.6) (layer "F.Cu") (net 2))
 (segment (start 166.41 134.45) (end 166.41 124.13) (width 0.6) (layer "F.Cu") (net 2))
 (segment (start 140.17 78.61) (end 140.17 92.645935) (width 0.6) (layer "F.Cu") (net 2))
 (segment (start 182.9 132.08) (end 181.95 132.08) (width 0.6) (layer "F.Cu") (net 2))
 (segment (start 136.49 131.02) (end 135.26 129.79) (width 0.6) (layer "F.Cu") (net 2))
 (segment (start 142.46 129.47) (end 141.47 128.48) (width 0.6) (layer "F.Cu") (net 7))
 (segment (start 152.56 92.18) (end 156.6 96.22) (width 0.6) (layer "F.Cu") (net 7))
 (segment (start 150.27 92.18) (end 150.27 82.865935) (width 0.6) (layer "F.Cu") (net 7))
 (segment (start 185.54 136.08) (end 181.4 140.22) (width 0.6) (layer "F.Cu") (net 7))
 (segment (start 140.725 134.575) (end 142.46 132.84) (width 0.6) (layer "F.Cu") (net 7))
 (segment (start 143.804065 95.185935) (end 140.17 95.185935) (width 0.6) (layer "F.Cu") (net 7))
 (segment (start 180.72 126.64) (end 180.72 128.38) (width 0.6) (layer "F.Cu") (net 7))
 (segment (start 142.64 109.89) (end 141.224065 111.305935) (width 0.6) (layer "F.Cu") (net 7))
 (segment (start 136.88 105.12) (end 137.86 106.1) (width 0.6) (layer "F.Cu") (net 7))
 (segment (start 138.07 128.48) (end 140.25 128.48) (width 0.6) (layer "F.Cu") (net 7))
 (segment (start 139.374065 95.185935) (end 136.88 97.68) (width 0.6) (layer "F.Cu") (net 7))
 (segment (start 140.13 111.305935) (end 138.494065 111.305935) (width 0.6) (layer "F.Cu") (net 7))
 (segment (start 150.27 92.18) (end 152.56 92.18) (width 0.6) (layer "F.Cu") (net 7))
 (segment (start 136.27 126.68) (end 138.07 128.48) (width 0.6) (layer "F.Cu") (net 7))
 (segment (start 142.64 107.29) (end 142.64 109.89) (width 0.6) (layer "F.Cu") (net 7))
 (segment (start 181.88 129.54) (end 184.06 129.54) (width 0.6) (layer "F.Cu") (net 7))
 (segment (start 182.78 118.84) (end 183.62 118.84) (width 0.6) (layer "F.Cu") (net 7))
 (segment (start 185.07 120.29) (end 185.07 122.29) (width 0.6) (layer "F.Cu") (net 7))
 (segment (start 183.62 118.84) (end 185.07 120.29) (width 0.6) (layer "F.Cu") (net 7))
 (segment (start 150.27 92.18) (end 146.81 92.18) (width 0.6) (layer "F.Cu") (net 7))
 (segment (start 181.4 140.22) (end 146.37 140.22) (width 0.6) (layer "F.Cu") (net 7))
 (segment (start 185.54 131.02) (end 185.54 136.08) (width 0.6) (layer "F.Cu") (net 7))
 (segment (start 141.224065 111.305935) (end 140.13 111.305935) (width 0.6) (layer "F.Cu") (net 7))
 (segment (start 142.46 132.84) (end 142.46 129.47) (width 0.6) (layer "F.Cu") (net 7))
 (segment (start 136.88 97.68) (end 136.88 105.12) (width 0.6) (layer "F.Cu") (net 7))
 (segment (start 146.81 92.18) (end 143.804065 95.185935) (width 0.6) (layer "F.Cu") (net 7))
 (segment (start 180.72 128.38) (end 181.88 129.54) (width 0.6) (layer "F.Cu") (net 7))
 (segment (start 184.06 129.54) (end 185.54 131.02) (width 0.6) (layer "F.Cu") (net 7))
 (segment (start 146.37 140.22) (end 140.725 134.575) (width 0.6) (layer "F.Cu") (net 7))
 (segment (start 150.27 82.865935) (end 150.59 82.545935) (width 0.6) (layer "F.Cu") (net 7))
 (segment (start 136.27 113.53) (end 136.27 126.68) (width 0.6) (layer "F.Cu") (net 7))
 (segment (start 138.494065 111.305935) (end 136.27 113.53) (width 0.6) (layer "F.Cu") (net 7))
 (segment (start 137.86 106.1) (end 141.45 106.1) (width 0.6) (layer "F.Cu") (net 7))
 (segment (start 156.6 96.22) (end 160.04 96.22) (width 0.6) (layer "F.Cu") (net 7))
 (segment (start 141.47 128.48) (end 140.25 128.48) (width 0.6) (layer "F.Cu") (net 7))
 (segment (start 185.07 122.29) (end 180.72 126.64) (width 0.6) (layer "F.Cu") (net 7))
 (segment (start 140.17 95.185935) (end 139.374065 95.185935) (width 0.6) (layer "F.Cu") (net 7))
 (segment (start 141.45 106.1) (end 142.64 107.29) (width 0.6) (layer "F.Cu") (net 7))
 (segment (start 147.55 117.58) (end 150.27 117.58) (width 0.6) (layer "F.Cu") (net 8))
 (segment (start 146.16 121.61) (end 146.16 118.97) (width 0.6) (layer "F.Cu") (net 8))
 (segment (start 143.07 122.51) (end 145.26 122.51) (width 0.6) (layer "F.Cu") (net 8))
 (segment (start 140.13 121.465935) (end 142.025935 121.465935) (width 0.6) (layer "F.Cu") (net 8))
 (segment (start 145.26 122.51) (end 146.16 121.61) (width 0.6) (layer "F.Cu") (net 8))
 (segment (start 142.025935 121.465935) (end 143.07 122.51) (width 0.6) (layer "F.Cu") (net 8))
 (segment (start 150.18 117.67) (end 150.27 117.58) (width 0.6) (layer "F.Cu") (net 8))
 (segment (start 146.16 118.97) (end 147.55 117.58) (width 0.6) (layer "F.Cu") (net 8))
 (segment (start 137.53 120.16) (end 137.53 122.19) (width 0.6) (layer "F.Cu") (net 9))
 (segment (start 138.764065 118.925935) (end 137.53 120.16) (width 0.6) (layer "F.Cu") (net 9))
 (segment (start 140.13 118.925935) (end 138.764065 118.925935) (width 0.6) (layer "F.Cu") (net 9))
 (segment (start 137.53 122.19) (end 139.03 123.69) (width 0.6) (layer "F.Cu") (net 9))
 (segment (start 139.03 123.69) (end 149.24 123.69) (width 0.6) (layer "F.Cu") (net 9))
 (segment (start 149.24 123.69) (end 150.27 122.66) (width 0.6) (layer "F.Cu") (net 9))
 (segment (start 167 78.07) (end 168.01 79.08) (width 0.6) (layer "F.Cu") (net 4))
 (segment (start 177.22 105.85) (end 175.47 107.6) (width 0.6) (layer "F.Cu") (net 4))
 (segment (start 162.85 78.04) (end 162.88 78.07) (width 0.6) (layer "F.Cu") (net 4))
 (segment (start 168.01 79.08) (end 168.01 82.95) (width 0.6) (layer "F.Cu") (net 4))
 (segment (start 168.01 82.95) (end 177.22 92.16) (width 0.6) (layer "F.Cu") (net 4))
 (segment (start 177.22 92.16) (end 177.22 105.85) (width 0.6) (layer "F.Cu") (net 4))
 (segment (start 165.98 78.07) (end 167 78.07) (width 0.6) (layer "F.Cu") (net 4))
 (segment (start 151.164065 78.04) (end 162.85 78.04) (width 0.6) (layer "F.Cu") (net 4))
 (segment (start 150.55 77.425935) (end 151.164065 78.04) (width 0.6) (layer "F.Cu") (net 4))
 (segment (start 175.47 107.6) (end 173.77 107.6) (width 0.6) (layer "F.Cu") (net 4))
 (segment (start 166.02 93.53) (end 168.19 95.7) (width 0.6) (layer "F.Cu") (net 3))
 (segment (start 151.394065 80.79) (end 162.78 80.79) (width 0.6) (layer "F.Cu") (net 3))
 (segment (start 166.02 80.93) (end 166.02 93.53) (width 0.6) (layer "F.Cu") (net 3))
 (segment (start 170.29 105.06) (end 173.77 105.06) (width 0.6) (layer "F.Cu") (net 3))
 (segment (start 162.78 80.79) (end 162.92 80.93) (width 0.6) (layer "F.Cu") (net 3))
 (segment (start 168.19 95.7) (end 168.19 102.96) (width 0.6) (layer "F.Cu") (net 3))
 (segment (start 150.59 79.985935) (end 151.394065 80.79) (width 0.6) (layer "F.Cu") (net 3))
 (segment (start 168.19 102.96) (end 170.29 105.06) (width 0.6) (layer "F.Cu") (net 3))
 (segment (start 177.7 117.79) (end 181.73 113.76) (width 0.6) (layer "F.Cu") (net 6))
 (segment (start 174.97 135.54) (end 173.77 135.54) (width 0.6) (layer "F.Cu") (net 6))
 (segment (start 181.73 113.76) (end 182.78 113.76) (width 0.6) (layer "F.Cu") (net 6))
 (segment (start 177.7 120.89) (end 177.7 132.81) (width 0.6) (layer "F.Cu") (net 6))
 (segment (start 177.7 132.81) (end 174.97 135.54) (width 0.6) (layer "F.Cu") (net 6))
 (segment (start 176.14 119.3) (end 178.94 119.3) (width 0.6) (layer "F.Cu") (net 23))
 (segment (start 173.77 120.3) (end 173.78 120.31) (width 0.6) (layer "F.Cu") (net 23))
 (segment (start 173.77 120.3) (end 175.14 120.3) (width 0.6) (layer "F.Cu") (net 23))
 (segment (start 181.94 116.3) (end 182.78 116.3) (width 0.6) (layer "F.Cu") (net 23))
 (segment (start 178.94 119.3) (end 181.94 116.3) (width 0.6) (layer "F.Cu") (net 23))
 (segment (start 175.14 120.3) (end 176.14 119.3) (width 0.6) (layer "F.Cu") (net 23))
 (segment (start 181.51 111.22) (end 182.78 111.22) (width 0.6) (layer "F.Cu") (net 24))
 (segment (start 174.97 117.76) (end 181.51 111.22) (width 0.6) (layer "F.Cu") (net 24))
 (segment (start 173.77 117.76) (end 174.97 117.76) (width 0.6) (layer "F.Cu") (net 24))
 (segment (start 174.62 115.22) (end 181.16 108.68) (width 0.6) (layer "F.Cu") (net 25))
 (segment (start 181.16 108.68) (end 182.78 108.68) (width 0.6) (layer "F.Cu") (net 25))
 (segment (start 173.77 115.22) (end 174.62 115.22) (width 0.6) (layer "F.Cu") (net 25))
 (segment (start 176.44 110.14) (end 173.77 110.14) (width 0.6) (layer "F.Cu") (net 26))
 (segment (start 182.9 126.9) (end 186.16 123.64) (width 0.6) (layer "F.Cu") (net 26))
 (segment (start 180.13 106.45) (end 176.44 110.14) (width 0.6) (layer "F.Cu") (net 26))
 (segment (start 184.42 106.45) (end 180.13 106.45) (width 0.6) (layer "F.Cu") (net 26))
 (segment (start 186.16 123.64) (end 186.16 108.19) (width 0.6) (layer "F.Cu") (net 26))
 (segment (start 186.16 108.19) (end 184.42 106.45) (width 0.6) (layer "F.Cu") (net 26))
 (segment (start 182.9 127) (end 182.9 126.9) (width 0.6) (layer "F.Cu") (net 26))
 (segment (start 140.25 125.94) (end 140.26 125.95) (width 0.6) (layer "F.Cu") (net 15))
 (segment (start 144.9 125.95) (end 146.69 127.74) (width 0.6) (layer "F.Cu") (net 15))
 (segment (start 140.26 125.95) (end 144.9 125.95) (width 0.6) (layer "F.Cu") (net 15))
 (segment (start 146.69 127.74) (end 150.27 127.74) (width 0.6) (layer "F.Cu") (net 15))
 (segment (start 144.924065 113.845935) (end 145.03 113.74) (width 0.6) (layer "F.Cu") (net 5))
 (segment (start 147.7 120.09) (end 150.24 120.09) (width 0.6) (layer "F.Cu") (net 5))
 (segment (start 144.89 116.98) (end 145.03 116.84) (width 0.6) (layer "F.Cu") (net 5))
 (segment (start 140.13 113.845935) (end 144.924065 113.845935) (width 0.6) (layer "F.Cu") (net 5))
 (segment (start 150.24 120.09) (end 150.27 120.12) (width 0.6) (layer "F.Cu") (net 5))
 (segment (start 144.89 119.8) (end 144.89 116.98) (width 0.6) (layer "F.Cu") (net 5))
 (segment (start 144.6 120.09) (end 144.89 119.8) (width 0.6) (layer "F.Cu") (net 5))
 (segment (start 149.93 115.38) (end 150.27 115.04) (width 0.6) (layer "F.Cu") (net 10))
 (segment (start 140.13 116.385935) (end 142.694065 116.385935) (width 0.6) (layer "F.Cu") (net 10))
 (segment (start 142.694065 116.385935) (end 143.7 115.38) (width 0.6) (layer "F.Cu") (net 10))
 (segment (start 143.7 115.38) (end 149.93 115.38) (width 0.6) (layer "F.Cu") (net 10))
 (segment (start 140.17 103.03) (end 149.64 112.5) (width 0.6) (layer "F.Cu") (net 13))
 (segment (start 140.17 102.805935) (end 140.17 103.03) (width 0.6) (layer "F.Cu") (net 13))
 (segment (start 149.64 112.5) (end 150.27 112.5) (width 0.6) (layer "F.Cu") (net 13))
 (segment (start 140.17 100.265935) (end 140.555935 100.265935) (width 0.6) (layer "F.Cu") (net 12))
 (segment (start 150.25 109.96) (end 150.27 109.96) (width 0.6) (layer "F.Cu") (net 12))
 (segment (start 140.555935 100.265935) (end 150.25 109.96) (width 0.6) (layer "F.Cu") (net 12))
 (segment (start 140.17 97.725935) (end 144.225935 97.725935) (width 0.6) (layer "F.Cu") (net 11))
 (segment (start 144.225935 97.725935) (end 148.84 102.34) (width 0.6) (layer "F.Cu") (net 11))
 (segment (start 148.84 102.34) (end 150.27 102.34) (width 0.6) (layer "F.Cu") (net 11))
 (segment (start 180.49 74.94) (end 182.72 74.94) (width 0.6) (layer "F.Cu") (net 18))
 (segment (start 177.605935 72.055935) (end 180.49 74.94) (width 0.6) (layer "F.Cu") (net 18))
 (segment (start 173.17 72.055935) (end 177.605935 72.055935) (width 0.6) (layer "F.Cu") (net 18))
 (segment (start 180.47 77.48) (end 182.72 77.48) (width 0.6) (layer "F.Cu") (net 19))
 (segment (start 173.16 74.645935) (end 177.635935 74.645935) (width 0.6) (layer "F.Cu") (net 19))
 (segment (start 177.635935 74.645935) (end 180.47 77.48) (width 0.6) (layer "F.Cu") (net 19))
 (segment (start 173.13 77.325935) (end 178.005935 77.325935) (width 0.6) (layer "F.Cu") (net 20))
 (segment (start 180.7 80.02) (end 182.72 80.02) (width 0.6) (layer "F.Cu") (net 20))
 (segment (start 178.005935 77.325935) (end 180.7 80.02) (width 0.6) (layer "F.Cu") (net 20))
 (segment (start 180.57 82.56) (end 182.72 82.56) (width 0.6) (layer "F.Cu") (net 21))
 (segment (start 177.925935 79.915935) (end 180.57 82.56) (width 0.6) (layer "F.Cu") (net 21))
 (segment (start 173.12 79.915935) (end 177.925935 79.915935) (width 0.6) (layer "F.Cu") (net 21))
 (segment (start 159.66 135.36) (end 159.71 135.41) (width 0.6) (layer "F.Cu") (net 1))
 (segment (start 150.27 135.36) (end 159.66 135.36) (width 0.6) (layer "F.Cu") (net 1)))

